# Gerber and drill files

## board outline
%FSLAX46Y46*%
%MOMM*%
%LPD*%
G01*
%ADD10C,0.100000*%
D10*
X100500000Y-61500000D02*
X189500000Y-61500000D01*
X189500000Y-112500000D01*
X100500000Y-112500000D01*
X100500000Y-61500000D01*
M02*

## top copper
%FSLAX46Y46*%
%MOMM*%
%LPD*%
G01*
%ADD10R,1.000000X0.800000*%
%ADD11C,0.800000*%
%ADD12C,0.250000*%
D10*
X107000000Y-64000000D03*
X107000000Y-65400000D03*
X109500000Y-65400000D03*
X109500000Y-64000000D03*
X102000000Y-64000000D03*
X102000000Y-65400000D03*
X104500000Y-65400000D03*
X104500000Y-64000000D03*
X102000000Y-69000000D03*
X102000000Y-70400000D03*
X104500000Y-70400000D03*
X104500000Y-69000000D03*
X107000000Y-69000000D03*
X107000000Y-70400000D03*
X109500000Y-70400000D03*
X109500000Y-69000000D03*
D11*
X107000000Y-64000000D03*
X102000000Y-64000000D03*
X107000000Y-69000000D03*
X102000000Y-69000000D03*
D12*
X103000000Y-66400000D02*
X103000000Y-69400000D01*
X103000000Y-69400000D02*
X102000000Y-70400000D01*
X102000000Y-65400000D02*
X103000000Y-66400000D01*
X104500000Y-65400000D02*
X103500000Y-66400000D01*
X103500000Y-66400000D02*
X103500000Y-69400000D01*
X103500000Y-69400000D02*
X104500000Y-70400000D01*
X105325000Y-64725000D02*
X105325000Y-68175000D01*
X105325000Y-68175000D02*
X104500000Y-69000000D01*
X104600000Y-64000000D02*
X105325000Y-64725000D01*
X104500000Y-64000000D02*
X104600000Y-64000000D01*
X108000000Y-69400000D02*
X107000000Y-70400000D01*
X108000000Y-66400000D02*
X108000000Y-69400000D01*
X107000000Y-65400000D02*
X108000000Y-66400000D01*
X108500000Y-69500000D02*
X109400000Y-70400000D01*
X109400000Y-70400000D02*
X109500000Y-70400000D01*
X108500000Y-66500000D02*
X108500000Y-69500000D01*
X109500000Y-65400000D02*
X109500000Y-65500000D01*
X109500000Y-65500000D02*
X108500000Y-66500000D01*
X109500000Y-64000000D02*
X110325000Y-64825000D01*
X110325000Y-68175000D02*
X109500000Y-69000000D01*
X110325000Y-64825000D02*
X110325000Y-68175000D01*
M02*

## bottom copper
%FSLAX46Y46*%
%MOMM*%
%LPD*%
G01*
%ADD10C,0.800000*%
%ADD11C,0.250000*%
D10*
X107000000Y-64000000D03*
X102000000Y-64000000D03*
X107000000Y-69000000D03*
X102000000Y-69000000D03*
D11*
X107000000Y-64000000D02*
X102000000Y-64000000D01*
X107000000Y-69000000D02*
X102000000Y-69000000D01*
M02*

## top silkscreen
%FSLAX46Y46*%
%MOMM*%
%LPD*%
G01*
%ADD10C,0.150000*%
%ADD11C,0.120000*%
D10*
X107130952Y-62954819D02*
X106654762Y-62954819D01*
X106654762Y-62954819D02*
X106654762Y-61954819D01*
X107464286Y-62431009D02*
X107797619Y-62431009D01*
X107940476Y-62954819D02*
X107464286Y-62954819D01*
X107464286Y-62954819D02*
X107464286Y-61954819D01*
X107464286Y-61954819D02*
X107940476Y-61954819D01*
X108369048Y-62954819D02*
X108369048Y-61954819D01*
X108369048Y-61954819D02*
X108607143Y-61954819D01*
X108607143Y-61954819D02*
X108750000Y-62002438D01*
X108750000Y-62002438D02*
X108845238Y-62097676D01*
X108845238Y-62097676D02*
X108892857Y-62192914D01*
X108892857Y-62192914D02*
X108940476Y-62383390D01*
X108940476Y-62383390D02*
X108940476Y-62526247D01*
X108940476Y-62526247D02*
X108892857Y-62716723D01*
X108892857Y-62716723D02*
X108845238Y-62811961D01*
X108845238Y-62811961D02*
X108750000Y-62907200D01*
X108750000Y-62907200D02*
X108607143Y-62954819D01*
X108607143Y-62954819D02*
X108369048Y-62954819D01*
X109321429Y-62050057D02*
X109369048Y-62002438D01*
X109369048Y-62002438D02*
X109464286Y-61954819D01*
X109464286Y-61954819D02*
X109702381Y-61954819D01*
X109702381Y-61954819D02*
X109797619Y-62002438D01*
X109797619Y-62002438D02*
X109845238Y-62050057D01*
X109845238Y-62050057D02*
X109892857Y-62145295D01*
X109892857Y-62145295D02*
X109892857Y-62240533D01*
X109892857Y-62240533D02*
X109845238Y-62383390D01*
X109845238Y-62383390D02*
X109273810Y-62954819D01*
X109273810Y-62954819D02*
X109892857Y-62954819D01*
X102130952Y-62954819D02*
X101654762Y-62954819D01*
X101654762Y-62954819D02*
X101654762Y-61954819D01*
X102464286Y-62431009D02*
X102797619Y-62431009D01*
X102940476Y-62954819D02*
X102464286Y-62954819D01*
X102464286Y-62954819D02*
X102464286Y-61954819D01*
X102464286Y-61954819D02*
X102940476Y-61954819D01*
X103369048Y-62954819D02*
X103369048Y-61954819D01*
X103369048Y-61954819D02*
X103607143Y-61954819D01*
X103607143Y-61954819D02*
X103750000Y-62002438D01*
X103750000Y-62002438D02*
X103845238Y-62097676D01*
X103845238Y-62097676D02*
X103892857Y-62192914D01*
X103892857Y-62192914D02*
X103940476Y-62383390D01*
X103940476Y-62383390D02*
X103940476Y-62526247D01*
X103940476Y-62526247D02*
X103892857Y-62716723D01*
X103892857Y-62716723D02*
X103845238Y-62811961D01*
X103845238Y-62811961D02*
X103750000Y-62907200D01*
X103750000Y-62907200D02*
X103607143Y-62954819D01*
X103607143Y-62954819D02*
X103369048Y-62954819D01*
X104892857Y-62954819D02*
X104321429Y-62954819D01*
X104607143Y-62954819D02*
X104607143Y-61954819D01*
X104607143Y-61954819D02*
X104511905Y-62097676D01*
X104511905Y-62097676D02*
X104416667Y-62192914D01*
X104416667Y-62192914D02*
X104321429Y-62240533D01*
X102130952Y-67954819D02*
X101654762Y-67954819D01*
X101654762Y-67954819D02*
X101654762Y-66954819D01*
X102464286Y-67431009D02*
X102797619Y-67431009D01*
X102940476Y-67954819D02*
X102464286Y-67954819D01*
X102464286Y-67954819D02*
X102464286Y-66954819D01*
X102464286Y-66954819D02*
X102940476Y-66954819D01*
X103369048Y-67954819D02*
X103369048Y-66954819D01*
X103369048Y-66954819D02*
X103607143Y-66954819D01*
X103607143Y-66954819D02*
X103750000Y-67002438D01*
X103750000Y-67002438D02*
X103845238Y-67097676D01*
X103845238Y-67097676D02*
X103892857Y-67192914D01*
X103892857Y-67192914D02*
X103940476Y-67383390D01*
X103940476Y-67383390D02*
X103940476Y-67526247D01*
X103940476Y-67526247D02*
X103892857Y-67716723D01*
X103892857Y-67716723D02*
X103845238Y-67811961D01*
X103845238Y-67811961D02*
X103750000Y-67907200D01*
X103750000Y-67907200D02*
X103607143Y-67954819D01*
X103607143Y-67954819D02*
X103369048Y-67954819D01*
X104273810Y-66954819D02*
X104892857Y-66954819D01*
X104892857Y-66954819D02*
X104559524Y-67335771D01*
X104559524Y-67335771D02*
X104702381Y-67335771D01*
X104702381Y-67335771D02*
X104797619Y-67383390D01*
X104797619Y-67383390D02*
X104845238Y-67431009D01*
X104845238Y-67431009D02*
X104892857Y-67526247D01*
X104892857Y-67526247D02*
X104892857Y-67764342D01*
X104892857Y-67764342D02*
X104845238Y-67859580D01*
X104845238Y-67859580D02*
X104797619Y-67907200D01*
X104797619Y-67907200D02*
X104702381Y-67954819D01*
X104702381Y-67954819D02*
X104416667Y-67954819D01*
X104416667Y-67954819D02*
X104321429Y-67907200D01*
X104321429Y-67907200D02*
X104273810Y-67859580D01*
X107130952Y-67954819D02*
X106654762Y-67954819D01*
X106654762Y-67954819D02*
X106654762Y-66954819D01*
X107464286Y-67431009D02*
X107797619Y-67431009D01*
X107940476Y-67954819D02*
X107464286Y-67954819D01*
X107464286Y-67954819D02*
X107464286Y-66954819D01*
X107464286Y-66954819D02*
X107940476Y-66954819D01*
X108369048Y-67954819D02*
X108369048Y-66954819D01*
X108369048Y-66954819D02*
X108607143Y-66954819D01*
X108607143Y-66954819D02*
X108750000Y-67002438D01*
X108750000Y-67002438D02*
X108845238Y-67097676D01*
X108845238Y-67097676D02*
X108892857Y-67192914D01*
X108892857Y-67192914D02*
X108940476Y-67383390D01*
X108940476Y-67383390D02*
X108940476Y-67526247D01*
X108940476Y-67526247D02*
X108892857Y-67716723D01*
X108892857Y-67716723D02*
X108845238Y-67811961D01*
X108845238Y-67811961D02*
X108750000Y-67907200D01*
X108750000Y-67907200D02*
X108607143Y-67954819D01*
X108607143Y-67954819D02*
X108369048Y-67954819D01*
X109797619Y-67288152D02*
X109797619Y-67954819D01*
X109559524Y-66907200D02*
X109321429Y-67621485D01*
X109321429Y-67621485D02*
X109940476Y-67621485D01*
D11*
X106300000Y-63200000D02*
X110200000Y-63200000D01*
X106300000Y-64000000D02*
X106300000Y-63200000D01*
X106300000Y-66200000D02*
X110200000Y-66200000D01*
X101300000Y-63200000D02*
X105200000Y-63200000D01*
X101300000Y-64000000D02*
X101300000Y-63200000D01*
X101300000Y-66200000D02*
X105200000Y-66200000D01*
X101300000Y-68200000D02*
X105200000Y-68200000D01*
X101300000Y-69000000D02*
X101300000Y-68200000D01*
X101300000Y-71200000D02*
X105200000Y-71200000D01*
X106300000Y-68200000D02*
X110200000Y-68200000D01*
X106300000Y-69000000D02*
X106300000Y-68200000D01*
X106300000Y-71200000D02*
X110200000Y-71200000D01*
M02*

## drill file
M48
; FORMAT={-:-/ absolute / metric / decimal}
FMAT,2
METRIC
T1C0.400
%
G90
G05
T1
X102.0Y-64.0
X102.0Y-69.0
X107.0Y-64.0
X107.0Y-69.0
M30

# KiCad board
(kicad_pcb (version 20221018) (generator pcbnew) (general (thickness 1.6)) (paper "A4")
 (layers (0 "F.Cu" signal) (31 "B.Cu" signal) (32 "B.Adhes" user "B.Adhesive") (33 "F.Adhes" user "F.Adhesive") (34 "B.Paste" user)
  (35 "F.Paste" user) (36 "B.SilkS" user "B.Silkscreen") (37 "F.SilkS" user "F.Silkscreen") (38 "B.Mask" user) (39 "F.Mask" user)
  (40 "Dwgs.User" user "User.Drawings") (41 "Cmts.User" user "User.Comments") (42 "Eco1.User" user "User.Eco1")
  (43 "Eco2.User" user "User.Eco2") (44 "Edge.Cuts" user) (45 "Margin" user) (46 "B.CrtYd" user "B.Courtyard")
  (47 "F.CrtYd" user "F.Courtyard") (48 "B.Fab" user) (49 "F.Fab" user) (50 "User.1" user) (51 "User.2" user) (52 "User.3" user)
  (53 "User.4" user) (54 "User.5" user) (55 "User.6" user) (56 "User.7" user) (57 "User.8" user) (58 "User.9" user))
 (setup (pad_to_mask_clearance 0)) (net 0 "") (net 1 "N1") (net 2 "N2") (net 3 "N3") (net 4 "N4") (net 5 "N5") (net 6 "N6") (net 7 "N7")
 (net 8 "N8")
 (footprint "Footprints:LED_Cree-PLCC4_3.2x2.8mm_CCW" (layer "F.Cu") (at 108.25 64.7)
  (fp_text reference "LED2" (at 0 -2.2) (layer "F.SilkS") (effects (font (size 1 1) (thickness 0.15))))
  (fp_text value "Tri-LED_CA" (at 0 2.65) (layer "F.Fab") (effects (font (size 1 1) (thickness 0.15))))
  (fp_line (start -1.95 -1.5) (end 1.95 -1.5) (stroke (width 0.12) (type solid)) (layer "F.SilkS"))
  (fp_line (start -1.95 -0.7) (end -1.95 -1.5) (stroke (width 0.12) (type solid)) (layer "F.SilkS"))
  (fp_line (start -1.95 1.5) (end 1.95 1.5) (stroke (width 0.12) (type solid)) (layer "F.SilkS"))
  (pad "1" smd rect (at -1.25 -0.7) (size 1 0.8) (layers "F.Cu" "F.Paste" "F.Mask") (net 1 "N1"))
  (pad "2" smd rect (at -1.25 0.7) (size 1 0.8) (layers "F.Cu" "F.Paste" "F.Mask") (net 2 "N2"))
  (pad "3" smd rect (at 1.25 0.7) (size 1 0.8) (layers "F.Cu" "F.Paste" "F.Mask") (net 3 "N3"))
  (pad "4" smd rect (at 1.25 -0.7) (size 1 0.8) (layers "F.Cu" "F.Paste" "F.Mask") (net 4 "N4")))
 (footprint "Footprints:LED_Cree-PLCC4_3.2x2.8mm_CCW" (layer "F.Cu") (at 103.25 64.7)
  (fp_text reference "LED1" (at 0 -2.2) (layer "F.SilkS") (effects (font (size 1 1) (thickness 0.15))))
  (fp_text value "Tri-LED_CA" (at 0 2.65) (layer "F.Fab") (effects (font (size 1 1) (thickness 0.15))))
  (fp_line (start -1.95 -1.5) (end 1.95 -1.5) (stroke (width 0.12) (type solid)) (layer "F.SilkS"))
  (fp_line (start -1.95 -0.7) (end -1.95 -1.5) (stroke (width 0.12) (type solid)) (layer "F.SilkS"))
  (fp_line (start -1.95 1.5) (end 1.95 1.5) (stroke (width 0.12) (type solid)) (layer "F.SilkS"))
  (pad "1" smd rect (at -1.25 -0.7) (size 1 0.8) (layers "F.Cu" "F.Paste" "F.Mask") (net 1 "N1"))
  (pad "2" smd rect (at -1.25 0.7) (size 1 0.8) (layers "F.Cu" "F.Paste" "F.Mask") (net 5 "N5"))
  (pad "3" smd rect (at 1.25 0.7) (size 1 0.8) (layers "F.Cu" "F.Paste" "F.Mask") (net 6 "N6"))
  (pad "4" smd rect (at 1.25 -0.7) (size 1 0.8) (layers "F.Cu" "F.Paste" "F.Mask") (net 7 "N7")))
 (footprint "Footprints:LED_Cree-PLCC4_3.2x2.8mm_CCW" (layer "F.Cu") (at 103.25 69.7)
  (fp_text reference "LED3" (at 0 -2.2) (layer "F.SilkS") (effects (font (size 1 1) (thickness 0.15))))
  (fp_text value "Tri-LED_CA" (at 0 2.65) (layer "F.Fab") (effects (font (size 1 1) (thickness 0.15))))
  (fp_line (start -1.95 -1.5) (end 1.95 -1.5) (stroke (width 0.12) (type solid)) (layer "F.SilkS"))
  (fp_line (start -1.95 -0.7) (end -1.95 -1.5) (stroke (width 0.12) (type solid)) (layer "F.SilkS"))
  (fp_line (start -1.95 1.5) (end 1.95 1.5) (stroke (width 0.12) (type solid)) (layer "F.SilkS"))
  (pad "1" smd rect (at -1.25 -0.7) (size 1 0.8) (layers "F.Cu" "F.Paste" "F.Mask") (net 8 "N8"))
  (pad "2" smd rect (at -1.25 0.7) (size 1 0.8) (layers "F.Cu" "F.Paste" "F.Mask") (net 5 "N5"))
  (pad "3" smd rect (at 1.25 0.7) (size 1 0.8) (layers "F.Cu" "F.Paste" "F.Mask") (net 6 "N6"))
  (pad "4" smd rect (at 1.25 -0.7) (size 1 0.8) (layers "F.Cu" "F.Paste" "F.Mask") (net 7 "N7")))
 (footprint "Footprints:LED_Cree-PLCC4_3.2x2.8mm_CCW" (layer "F.Cu") (at 108.25 69.7)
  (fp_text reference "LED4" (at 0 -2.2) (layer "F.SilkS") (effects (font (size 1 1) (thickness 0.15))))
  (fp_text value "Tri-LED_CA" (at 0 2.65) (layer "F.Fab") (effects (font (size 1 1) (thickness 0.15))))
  (fp_line (start -1.95 -1.5) (end 1.95 -1.5) (stroke (width 0.12) (type solid)) (layer "F.SilkS"))
  (fp_line (start -1.95 -0.7) (end -1.95 -1.5) (stroke (width 0.12) (type solid)) (layer "F.SilkS"))
  (fp_line (start -1.95 1.5) (end 1.95 1.5) (stroke (width 0.12) (type solid)) (layer "F.SilkS"))
  (pad "1" smd rect (at -1.25 -0.7) (size 1 0.8) (layers "F.Cu" "F.Paste" "F.Mask") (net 8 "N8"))
  (pad "2" smd rect (at -1.25 0.7) (size 1 0.8) (layers "F.Cu" "F.Paste" "F.Mask") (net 2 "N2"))
  (pad "3" smd rect (at 1.25 0.7) (size 1 0.8) (layers "F.Cu" "F.Paste" "F.Mask") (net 3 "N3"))
  (pad "4" smd rect (at 1.25 -0.7) (size 1 0.8) (layers "F.Cu" "F.Paste" "F.Mask") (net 4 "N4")))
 (gr_rect (start 100.5 61.5) (end 189.5 112.5) (stroke (width 0.1) (type default)) (fill none) (layer "Edge.Cuts"))
 (via (at 107 64) (size 0.8) (drill 0.4) (layers "F.Cu" "B.Cu") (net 1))
 (via (at 102 64) (size 0.8) (drill 0.4) (layers "F.Cu" "B.Cu") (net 1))
 (segment (start 107 64) (end 102 64) (width 0.25) (layer "B.Cu") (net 1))
 (segment (start 103 66.4) (end 103 69.4) (width 0.25) (layer "F.Cu") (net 5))
 (segment (start 103 69.4) (end 102 70.4) (width 0.25) (layer "F.Cu") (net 5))
 (segment (start 102 65.4) (end 103 66.4) (width 0.25) (layer "F.Cu") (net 5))
 (segment (start 104.5 65.4) (end 103.5 66.4) (width 0.25) (layer "F.Cu") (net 6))
 (segment (start 103.5 66.4) (end 103.5 69.4) (width 0.25) (layer "F.Cu") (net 6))
 (segment (start 103.5 69.4) (end 104.5 70.4) (width 0.25) (layer "F.Cu") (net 6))
 (segment (start 105.325 64.725) (end 105.325 68.175) (width 0.25) (layer "F.Cu") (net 7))
 (segment (start 105.325 68.175) (end 104.5 69) (width 0.25) (layer "F.Cu") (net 7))
 (segment (start 104.6 64) (end 105.325 64.725) (width 0.25) (layer "F.Cu") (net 7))
 (segment (start 104.5 64) (end 104.6 64) (width 0.25) (layer "F.Cu") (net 7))
 (segment (start 108 69.4) (end 107 70.4) (width 0.25) (layer "F.Cu") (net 2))
 (segment (start 108 66.4) (end 108 69.4) (width 0.25) (layer "F.Cu") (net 2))
 (segment (start 107 65.4) (end 108 66.4) (width 0.25) (layer "F.Cu") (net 2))
 (segment (start 108.5 69.5) (end 109.4 70.4) (width 0.25) (layer "F.Cu") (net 3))
 (segment (start 109.4 70.4) (end 109.5 70.4) (width 0.25) (layer "F.Cu") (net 3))
 (segment (start 108.5 66.5) (end 108.5 69.5) (width 0.25) (layer "F.Cu") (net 3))
 (segment (start 109.5 65.4) (end 109.5 65.5) (width 0.25) (layer "F.Cu") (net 3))
 (segment (start 109.5 65.5) (end 108.5 66.5) (width 0.25) (layer "F.Cu") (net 3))
 (segment (start 109.5 64) (end 110.325 64.825) (width 0.25) (layer "F.Cu") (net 4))
 (segment (start 110.325 68.175) (end 109.5 69) (width 0.25) (layer "F.Cu") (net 4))
 (segment (start 110.325 64.825) (end 110.325 68.175) (width 0.25) (layer "F.Cu") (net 4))
 (via (at 107 69) (size 0.8) (drill 0.4) (layers "F.Cu" "B.Cu") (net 8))
 (via (at 102 69) (size 0.8) (drill 0.4) (layers "F.Cu" "B.Cu") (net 8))
 (segment (start 107 69) (end 102 69) (width 0.25) (layer "B.Cu") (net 8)))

